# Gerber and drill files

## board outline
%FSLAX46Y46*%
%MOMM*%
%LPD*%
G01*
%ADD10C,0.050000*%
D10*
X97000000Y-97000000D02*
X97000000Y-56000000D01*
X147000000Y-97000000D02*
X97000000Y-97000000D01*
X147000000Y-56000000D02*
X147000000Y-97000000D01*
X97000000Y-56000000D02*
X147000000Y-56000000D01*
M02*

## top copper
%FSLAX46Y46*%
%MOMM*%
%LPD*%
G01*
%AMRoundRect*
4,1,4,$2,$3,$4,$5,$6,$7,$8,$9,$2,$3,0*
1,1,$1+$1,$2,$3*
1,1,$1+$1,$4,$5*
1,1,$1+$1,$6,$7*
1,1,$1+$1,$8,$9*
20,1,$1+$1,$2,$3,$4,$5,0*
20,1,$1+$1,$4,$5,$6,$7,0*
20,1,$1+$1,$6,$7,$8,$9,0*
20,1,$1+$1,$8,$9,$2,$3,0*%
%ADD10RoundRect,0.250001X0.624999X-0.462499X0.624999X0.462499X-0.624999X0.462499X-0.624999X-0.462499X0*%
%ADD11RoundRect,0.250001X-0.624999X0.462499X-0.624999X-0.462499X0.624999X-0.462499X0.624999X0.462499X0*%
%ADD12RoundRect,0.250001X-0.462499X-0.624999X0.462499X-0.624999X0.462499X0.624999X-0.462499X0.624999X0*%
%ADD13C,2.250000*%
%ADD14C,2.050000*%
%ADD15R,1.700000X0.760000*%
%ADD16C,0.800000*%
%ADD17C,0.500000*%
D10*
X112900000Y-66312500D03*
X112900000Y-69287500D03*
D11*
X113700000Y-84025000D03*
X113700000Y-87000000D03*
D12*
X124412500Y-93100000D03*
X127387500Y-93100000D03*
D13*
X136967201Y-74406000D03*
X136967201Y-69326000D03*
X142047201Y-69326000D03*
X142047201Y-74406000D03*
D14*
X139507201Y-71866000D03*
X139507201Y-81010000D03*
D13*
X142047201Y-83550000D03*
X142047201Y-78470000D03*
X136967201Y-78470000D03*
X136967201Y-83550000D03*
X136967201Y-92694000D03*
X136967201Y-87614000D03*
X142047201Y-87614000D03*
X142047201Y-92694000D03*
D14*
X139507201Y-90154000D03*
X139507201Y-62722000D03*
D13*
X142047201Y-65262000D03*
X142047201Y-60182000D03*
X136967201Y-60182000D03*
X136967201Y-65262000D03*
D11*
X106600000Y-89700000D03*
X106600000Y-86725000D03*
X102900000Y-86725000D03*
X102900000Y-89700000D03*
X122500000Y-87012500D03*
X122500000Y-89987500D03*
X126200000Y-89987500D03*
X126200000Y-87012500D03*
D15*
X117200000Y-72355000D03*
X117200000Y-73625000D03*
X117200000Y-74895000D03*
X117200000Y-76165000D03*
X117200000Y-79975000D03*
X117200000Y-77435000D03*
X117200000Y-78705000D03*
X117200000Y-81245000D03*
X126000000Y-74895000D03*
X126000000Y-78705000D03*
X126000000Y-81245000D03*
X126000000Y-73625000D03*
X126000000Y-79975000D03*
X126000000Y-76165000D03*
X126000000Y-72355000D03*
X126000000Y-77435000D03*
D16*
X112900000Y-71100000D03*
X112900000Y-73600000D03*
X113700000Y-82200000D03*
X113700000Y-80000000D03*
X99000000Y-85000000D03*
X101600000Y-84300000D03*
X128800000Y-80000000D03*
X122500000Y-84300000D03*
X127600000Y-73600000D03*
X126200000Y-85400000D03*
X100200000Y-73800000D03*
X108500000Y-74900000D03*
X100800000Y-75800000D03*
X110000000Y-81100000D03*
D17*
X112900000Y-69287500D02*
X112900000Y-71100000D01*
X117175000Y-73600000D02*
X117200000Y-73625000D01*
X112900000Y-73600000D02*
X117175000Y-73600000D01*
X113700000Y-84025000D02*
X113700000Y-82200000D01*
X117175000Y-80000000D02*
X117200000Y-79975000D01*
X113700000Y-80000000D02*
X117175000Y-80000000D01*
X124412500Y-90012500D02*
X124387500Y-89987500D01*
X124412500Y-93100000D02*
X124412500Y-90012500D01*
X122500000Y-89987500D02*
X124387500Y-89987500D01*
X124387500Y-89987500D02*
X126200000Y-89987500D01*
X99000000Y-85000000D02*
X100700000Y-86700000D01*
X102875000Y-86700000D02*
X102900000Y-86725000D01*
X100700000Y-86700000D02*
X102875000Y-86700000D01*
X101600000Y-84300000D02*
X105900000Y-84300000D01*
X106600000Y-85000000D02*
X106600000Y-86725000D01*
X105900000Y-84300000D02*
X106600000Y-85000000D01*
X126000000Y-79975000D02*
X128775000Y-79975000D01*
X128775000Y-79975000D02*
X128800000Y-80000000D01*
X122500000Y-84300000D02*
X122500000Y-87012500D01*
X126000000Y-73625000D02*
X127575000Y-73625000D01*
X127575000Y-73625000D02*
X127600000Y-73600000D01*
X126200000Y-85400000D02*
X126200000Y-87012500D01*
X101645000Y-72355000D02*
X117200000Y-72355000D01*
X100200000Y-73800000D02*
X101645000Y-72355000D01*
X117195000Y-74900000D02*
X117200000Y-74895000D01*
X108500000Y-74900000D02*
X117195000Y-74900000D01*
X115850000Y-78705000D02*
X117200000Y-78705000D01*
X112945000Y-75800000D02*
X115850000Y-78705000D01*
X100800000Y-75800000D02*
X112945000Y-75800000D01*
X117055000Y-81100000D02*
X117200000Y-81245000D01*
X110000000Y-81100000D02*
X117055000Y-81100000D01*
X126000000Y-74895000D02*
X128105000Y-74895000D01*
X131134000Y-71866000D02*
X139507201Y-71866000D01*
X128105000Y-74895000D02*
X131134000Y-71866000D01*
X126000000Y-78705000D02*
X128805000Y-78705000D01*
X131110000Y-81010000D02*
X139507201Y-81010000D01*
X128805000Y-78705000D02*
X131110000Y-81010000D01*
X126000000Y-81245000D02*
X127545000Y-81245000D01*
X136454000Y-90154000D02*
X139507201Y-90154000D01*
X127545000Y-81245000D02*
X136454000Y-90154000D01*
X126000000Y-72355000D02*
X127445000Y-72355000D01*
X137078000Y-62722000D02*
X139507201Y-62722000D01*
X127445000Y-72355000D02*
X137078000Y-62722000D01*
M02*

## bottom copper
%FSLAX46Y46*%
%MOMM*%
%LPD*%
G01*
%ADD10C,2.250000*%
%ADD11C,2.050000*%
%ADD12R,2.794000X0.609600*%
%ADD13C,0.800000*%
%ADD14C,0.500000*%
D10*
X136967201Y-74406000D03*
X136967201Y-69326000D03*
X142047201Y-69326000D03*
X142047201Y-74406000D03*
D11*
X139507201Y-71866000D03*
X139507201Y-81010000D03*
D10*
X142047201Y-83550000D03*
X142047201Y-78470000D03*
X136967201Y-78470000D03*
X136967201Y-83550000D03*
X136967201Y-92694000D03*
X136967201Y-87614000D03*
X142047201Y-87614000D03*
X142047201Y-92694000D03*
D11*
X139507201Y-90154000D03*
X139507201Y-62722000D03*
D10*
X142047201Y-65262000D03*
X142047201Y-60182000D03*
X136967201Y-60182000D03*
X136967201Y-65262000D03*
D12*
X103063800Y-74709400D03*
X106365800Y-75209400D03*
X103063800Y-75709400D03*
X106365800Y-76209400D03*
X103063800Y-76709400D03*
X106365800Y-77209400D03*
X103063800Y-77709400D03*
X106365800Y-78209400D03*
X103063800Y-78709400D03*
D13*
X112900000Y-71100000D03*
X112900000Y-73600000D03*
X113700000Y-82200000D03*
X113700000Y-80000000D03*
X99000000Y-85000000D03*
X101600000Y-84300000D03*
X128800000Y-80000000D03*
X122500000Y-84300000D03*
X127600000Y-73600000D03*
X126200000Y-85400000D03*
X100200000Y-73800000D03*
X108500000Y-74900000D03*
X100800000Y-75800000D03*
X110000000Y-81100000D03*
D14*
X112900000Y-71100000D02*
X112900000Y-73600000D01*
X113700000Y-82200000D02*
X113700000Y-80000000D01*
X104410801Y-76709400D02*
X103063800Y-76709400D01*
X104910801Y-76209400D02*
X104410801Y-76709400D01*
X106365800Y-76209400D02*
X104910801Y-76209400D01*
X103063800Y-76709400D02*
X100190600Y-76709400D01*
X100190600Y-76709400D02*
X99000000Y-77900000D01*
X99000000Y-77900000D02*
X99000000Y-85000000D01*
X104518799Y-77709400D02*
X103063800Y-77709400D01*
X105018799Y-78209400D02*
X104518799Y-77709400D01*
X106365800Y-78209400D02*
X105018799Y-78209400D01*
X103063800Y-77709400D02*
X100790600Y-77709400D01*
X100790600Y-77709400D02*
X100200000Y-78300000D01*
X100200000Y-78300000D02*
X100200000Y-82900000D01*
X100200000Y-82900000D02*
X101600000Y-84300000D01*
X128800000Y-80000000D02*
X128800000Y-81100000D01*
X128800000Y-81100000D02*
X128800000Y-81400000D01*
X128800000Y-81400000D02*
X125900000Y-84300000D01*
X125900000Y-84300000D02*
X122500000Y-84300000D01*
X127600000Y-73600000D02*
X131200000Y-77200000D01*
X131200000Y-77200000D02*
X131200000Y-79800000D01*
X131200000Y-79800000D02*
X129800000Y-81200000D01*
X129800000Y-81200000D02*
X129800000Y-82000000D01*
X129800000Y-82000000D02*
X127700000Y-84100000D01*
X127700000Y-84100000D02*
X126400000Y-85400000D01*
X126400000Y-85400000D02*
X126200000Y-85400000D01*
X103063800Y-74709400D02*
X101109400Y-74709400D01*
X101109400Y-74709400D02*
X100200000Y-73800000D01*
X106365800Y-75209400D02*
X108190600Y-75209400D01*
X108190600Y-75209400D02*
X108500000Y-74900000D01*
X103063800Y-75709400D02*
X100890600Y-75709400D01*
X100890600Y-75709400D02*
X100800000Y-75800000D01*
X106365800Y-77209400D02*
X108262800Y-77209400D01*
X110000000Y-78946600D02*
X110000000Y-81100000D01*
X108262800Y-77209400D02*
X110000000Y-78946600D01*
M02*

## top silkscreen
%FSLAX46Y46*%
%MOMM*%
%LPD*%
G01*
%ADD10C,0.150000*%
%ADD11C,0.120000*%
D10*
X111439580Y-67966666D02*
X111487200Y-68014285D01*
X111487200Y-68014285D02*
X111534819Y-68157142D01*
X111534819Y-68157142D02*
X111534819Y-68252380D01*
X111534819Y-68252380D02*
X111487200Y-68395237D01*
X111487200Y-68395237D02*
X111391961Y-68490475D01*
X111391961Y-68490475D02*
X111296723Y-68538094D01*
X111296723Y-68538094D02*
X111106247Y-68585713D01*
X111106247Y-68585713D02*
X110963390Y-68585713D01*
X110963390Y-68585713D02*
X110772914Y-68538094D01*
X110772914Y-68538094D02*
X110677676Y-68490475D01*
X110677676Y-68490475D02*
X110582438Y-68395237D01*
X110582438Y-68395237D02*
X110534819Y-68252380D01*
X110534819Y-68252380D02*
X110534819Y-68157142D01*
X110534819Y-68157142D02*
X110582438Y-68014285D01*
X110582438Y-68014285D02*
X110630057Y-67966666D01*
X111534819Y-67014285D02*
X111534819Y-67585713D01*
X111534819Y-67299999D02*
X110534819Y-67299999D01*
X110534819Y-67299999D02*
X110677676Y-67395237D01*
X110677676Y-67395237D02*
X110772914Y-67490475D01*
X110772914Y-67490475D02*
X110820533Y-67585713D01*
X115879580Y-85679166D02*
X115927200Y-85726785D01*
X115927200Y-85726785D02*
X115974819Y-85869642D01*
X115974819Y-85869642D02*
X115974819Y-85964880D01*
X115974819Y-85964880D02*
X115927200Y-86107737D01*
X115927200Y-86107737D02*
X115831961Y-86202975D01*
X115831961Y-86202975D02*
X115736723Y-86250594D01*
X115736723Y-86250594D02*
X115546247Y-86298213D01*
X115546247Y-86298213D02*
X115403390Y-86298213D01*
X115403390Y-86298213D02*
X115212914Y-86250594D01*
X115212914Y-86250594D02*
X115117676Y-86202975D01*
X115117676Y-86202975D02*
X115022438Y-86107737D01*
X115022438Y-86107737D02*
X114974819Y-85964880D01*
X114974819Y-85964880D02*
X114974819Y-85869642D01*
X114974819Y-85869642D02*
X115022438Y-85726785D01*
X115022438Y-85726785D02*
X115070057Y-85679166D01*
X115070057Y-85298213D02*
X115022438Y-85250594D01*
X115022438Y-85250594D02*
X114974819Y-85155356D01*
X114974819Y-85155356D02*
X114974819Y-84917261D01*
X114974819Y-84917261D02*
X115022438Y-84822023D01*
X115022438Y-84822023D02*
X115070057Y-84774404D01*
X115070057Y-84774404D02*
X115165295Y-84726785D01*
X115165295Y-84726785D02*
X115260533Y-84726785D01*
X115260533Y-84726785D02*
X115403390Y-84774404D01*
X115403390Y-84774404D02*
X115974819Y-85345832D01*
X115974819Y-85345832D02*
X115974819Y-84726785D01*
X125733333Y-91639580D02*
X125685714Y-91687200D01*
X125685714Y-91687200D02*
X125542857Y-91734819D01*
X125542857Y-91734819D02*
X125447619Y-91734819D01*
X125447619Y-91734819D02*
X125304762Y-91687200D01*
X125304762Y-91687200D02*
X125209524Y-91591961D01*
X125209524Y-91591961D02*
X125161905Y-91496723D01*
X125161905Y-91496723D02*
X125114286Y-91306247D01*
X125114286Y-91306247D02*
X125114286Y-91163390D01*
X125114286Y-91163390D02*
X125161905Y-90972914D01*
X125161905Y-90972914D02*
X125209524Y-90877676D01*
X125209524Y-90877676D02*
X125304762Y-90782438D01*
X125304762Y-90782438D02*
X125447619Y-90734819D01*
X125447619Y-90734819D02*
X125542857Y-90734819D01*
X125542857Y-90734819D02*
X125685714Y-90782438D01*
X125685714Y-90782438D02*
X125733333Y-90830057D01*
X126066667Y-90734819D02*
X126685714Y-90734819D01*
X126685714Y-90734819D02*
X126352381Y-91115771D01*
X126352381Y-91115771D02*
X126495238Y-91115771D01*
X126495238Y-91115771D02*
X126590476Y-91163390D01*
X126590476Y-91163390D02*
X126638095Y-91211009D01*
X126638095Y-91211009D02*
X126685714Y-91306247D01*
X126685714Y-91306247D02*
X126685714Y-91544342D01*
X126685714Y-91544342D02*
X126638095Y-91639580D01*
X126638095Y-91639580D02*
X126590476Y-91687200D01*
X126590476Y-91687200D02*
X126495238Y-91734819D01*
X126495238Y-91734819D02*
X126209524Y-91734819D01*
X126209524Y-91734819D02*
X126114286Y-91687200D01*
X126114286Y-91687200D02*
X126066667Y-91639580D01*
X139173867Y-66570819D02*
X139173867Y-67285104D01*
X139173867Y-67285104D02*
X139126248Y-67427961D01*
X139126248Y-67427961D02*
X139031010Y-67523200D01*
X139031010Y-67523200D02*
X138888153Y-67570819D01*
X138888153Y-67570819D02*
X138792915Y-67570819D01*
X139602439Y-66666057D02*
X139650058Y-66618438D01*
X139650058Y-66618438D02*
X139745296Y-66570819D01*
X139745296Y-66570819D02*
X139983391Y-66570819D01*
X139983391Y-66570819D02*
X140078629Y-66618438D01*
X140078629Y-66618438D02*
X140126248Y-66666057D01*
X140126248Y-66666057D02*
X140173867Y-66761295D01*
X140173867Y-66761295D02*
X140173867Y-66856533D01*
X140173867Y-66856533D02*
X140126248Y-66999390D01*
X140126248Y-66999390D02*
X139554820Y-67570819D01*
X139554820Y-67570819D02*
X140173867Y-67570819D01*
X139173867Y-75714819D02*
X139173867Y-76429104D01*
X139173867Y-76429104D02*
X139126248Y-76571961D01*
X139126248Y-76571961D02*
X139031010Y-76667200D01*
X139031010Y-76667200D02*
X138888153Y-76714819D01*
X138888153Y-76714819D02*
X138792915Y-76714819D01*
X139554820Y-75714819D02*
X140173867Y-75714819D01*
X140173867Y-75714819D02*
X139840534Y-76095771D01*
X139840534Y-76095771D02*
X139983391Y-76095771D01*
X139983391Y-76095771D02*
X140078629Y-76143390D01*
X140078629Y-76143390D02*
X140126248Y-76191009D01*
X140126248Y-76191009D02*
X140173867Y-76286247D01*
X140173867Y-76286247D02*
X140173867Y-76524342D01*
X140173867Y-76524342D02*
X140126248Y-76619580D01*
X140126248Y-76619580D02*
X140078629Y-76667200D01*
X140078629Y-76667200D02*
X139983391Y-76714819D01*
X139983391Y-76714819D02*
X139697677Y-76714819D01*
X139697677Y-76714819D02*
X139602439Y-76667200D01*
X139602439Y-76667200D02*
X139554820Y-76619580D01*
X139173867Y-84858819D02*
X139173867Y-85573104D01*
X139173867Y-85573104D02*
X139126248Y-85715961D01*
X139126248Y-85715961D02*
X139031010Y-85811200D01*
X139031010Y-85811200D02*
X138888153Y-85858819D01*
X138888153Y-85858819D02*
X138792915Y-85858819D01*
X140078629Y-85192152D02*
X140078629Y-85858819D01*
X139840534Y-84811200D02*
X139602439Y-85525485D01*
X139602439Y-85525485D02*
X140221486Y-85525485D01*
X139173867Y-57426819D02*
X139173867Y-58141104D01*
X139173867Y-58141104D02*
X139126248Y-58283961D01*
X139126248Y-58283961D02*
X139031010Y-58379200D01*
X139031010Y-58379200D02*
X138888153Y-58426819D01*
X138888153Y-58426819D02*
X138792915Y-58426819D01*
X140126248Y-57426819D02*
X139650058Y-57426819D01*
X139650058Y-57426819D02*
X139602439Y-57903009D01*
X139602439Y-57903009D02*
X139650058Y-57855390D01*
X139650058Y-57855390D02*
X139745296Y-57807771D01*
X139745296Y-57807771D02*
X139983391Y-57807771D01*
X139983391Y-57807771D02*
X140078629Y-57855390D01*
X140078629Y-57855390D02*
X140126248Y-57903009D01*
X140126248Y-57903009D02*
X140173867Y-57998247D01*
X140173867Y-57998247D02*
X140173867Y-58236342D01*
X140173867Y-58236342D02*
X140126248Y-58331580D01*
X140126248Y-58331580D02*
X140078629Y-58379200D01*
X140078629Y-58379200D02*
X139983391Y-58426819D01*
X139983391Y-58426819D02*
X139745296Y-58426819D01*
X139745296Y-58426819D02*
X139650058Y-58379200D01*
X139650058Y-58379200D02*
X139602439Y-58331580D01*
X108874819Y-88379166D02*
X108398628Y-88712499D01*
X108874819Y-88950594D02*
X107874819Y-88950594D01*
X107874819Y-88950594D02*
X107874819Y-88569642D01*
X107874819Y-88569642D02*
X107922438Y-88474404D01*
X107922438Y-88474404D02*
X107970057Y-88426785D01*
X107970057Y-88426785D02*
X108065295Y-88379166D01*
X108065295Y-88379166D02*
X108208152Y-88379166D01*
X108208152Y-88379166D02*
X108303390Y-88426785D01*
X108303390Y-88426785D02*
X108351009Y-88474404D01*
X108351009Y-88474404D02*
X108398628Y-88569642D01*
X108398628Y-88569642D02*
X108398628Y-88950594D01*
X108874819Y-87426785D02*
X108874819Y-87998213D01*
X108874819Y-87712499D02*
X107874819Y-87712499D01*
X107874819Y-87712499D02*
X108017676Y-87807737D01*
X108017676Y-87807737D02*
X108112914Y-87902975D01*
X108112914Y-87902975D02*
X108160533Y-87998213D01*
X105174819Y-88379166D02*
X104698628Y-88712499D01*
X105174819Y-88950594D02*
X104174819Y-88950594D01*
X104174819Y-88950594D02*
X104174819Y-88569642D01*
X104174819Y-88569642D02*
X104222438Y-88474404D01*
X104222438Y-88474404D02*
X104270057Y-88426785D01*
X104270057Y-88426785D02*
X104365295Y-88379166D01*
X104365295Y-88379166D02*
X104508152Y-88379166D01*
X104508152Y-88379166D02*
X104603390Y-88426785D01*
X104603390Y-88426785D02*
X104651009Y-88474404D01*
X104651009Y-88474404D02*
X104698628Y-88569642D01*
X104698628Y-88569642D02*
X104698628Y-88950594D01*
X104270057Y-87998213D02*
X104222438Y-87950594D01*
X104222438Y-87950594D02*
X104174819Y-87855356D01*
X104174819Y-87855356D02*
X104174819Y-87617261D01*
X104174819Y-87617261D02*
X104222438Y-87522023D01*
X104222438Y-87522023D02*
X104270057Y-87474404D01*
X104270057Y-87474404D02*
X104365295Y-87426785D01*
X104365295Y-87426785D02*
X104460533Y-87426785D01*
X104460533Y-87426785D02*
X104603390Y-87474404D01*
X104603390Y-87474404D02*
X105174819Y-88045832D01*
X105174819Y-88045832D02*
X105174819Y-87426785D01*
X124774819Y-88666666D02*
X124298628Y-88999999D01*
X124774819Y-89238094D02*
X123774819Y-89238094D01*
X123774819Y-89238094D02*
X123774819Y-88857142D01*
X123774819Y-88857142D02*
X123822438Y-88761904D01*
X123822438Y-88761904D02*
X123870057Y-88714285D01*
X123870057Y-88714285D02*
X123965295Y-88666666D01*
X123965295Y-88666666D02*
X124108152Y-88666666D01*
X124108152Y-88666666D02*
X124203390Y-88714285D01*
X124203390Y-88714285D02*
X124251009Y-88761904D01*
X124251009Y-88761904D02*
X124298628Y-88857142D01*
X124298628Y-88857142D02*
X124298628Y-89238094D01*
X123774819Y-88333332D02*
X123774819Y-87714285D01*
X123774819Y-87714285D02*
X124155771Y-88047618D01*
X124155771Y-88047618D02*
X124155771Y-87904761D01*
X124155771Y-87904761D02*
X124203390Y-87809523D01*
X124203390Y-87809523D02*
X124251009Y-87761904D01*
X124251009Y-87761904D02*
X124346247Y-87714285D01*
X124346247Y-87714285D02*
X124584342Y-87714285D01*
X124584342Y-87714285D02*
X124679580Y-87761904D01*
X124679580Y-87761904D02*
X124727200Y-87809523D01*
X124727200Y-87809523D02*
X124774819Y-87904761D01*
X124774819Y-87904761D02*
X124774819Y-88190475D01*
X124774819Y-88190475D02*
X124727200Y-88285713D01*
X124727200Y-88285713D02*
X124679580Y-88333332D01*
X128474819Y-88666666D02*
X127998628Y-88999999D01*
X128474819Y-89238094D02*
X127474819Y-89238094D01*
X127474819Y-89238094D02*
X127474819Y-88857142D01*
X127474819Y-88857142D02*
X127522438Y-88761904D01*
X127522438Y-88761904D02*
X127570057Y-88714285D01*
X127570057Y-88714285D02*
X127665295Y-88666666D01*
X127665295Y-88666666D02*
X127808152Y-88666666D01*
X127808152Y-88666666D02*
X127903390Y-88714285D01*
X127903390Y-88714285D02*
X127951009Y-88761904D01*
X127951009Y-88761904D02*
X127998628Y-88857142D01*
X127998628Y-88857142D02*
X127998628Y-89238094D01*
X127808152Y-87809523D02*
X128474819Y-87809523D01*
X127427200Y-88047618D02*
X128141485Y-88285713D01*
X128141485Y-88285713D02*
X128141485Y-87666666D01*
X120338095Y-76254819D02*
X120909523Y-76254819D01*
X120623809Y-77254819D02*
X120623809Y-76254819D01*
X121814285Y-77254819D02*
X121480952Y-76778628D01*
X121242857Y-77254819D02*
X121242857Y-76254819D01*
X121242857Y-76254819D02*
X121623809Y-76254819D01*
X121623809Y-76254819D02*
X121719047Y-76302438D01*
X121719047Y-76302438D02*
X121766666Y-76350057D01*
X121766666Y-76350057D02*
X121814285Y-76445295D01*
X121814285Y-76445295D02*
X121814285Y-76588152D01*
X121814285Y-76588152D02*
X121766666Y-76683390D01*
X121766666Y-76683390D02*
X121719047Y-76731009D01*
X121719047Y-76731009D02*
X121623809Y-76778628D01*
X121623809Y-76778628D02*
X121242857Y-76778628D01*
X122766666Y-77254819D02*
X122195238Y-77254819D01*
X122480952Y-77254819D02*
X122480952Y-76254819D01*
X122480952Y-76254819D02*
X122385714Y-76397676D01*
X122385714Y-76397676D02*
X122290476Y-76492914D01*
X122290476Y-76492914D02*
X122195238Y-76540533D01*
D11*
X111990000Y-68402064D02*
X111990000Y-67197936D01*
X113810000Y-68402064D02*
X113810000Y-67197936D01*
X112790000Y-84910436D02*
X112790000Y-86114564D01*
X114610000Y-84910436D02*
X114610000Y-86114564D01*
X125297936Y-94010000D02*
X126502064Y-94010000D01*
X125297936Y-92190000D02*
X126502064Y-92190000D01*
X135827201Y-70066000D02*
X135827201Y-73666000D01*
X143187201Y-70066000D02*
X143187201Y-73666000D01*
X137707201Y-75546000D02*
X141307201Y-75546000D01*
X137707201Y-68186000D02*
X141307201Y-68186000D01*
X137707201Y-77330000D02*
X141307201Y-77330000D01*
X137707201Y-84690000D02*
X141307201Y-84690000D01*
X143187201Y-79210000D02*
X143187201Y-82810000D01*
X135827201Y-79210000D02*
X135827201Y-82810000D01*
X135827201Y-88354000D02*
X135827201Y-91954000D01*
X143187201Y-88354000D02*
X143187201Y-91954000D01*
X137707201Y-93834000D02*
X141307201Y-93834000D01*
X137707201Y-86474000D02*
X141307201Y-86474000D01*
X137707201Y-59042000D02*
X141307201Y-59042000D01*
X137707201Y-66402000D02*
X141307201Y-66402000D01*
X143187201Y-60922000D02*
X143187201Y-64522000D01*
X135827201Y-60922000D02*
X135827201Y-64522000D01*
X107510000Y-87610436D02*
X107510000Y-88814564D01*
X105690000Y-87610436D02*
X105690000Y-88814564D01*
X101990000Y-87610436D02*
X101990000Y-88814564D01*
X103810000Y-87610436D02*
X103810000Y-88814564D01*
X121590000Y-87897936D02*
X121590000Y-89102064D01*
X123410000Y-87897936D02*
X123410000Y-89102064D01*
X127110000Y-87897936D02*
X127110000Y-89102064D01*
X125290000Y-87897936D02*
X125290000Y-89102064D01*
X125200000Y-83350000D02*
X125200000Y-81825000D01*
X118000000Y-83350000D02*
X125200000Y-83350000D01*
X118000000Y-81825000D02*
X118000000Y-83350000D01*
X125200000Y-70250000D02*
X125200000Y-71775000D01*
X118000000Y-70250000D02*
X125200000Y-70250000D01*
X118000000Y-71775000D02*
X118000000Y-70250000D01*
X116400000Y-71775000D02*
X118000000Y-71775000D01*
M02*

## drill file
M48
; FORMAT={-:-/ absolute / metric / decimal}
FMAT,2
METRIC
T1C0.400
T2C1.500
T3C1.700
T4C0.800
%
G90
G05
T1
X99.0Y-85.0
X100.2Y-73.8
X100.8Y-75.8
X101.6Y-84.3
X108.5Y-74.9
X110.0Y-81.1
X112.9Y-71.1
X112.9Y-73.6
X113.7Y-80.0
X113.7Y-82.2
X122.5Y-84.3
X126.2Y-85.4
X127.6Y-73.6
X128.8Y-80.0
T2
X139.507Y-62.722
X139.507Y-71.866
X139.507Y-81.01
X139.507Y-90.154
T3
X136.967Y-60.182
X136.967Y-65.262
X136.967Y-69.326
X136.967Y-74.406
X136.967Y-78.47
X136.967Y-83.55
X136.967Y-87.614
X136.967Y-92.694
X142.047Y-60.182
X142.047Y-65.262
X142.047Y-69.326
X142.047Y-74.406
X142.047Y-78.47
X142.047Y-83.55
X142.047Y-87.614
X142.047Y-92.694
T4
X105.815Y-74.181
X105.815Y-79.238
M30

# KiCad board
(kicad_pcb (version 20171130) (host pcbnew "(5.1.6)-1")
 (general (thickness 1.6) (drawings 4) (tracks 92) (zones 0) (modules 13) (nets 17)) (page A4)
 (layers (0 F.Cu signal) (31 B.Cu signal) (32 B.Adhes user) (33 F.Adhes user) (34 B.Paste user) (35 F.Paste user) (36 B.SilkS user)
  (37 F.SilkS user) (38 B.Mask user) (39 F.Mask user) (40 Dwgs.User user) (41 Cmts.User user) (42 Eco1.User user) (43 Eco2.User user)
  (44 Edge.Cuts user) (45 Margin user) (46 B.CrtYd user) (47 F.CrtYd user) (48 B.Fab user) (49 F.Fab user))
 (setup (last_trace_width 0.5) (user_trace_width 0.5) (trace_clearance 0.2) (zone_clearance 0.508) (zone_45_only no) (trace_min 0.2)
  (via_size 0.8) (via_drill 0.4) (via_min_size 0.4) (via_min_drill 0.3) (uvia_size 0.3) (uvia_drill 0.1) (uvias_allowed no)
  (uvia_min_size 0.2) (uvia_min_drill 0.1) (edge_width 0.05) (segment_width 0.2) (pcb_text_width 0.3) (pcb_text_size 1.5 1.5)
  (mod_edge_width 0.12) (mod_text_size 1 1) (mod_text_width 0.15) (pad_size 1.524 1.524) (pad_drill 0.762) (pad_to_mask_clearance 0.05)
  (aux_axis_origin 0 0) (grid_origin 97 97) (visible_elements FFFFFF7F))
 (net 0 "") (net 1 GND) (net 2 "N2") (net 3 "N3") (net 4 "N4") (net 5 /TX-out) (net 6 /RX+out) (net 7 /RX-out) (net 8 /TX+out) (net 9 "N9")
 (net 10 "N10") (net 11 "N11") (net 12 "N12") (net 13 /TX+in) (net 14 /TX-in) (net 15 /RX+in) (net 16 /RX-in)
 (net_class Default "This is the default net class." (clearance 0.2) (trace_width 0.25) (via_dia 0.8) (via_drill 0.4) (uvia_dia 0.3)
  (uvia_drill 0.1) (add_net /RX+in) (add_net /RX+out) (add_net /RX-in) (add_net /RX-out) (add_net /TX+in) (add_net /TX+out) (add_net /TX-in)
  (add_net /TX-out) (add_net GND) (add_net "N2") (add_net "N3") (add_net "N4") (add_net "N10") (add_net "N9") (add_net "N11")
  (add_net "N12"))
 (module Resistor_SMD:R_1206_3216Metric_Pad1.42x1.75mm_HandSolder (layer F.Cu) (at 112.9 67.8 90)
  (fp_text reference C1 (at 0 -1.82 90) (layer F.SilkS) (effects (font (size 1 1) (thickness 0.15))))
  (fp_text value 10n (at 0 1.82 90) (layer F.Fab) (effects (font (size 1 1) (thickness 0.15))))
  (fp_line (start -0.602064 -0.91) (end 0.602064 -0.91) (layer F.SilkS) (width 0.12))
  (fp_line (start -0.602064 0.91) (end 0.602064 0.91) (layer F.SilkS) (width 0.12))
  (pad 2 smd roundrect (at 1.4875 0 90) (size 1.425 1.75) (layers F.Cu F.Paste F.Mask) (roundrect_rratio 0.175439) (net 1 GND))
  (pad 1 smd roundrect (at -1.4875 0 90) (size 1.425 1.75) (layers F.Cu F.Paste F.Mask) (roundrect_rratio 0.175439) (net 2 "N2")))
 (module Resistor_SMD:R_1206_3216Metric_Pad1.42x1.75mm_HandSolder (layer F.Cu) (at 113.7 85.5125 270)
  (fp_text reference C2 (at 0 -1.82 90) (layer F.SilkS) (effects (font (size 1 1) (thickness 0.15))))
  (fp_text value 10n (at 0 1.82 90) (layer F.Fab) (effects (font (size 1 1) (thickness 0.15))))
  (fp_line (start -0.602064 0.91) (end 0.602064 0.91) (layer F.SilkS) (width 0.12))
  (fp_line (start -0.602064 -0.91) (end 0.602064 -0.91) (layer F.SilkS) (width 0.12))
  (pad 1 smd roundrect (at -1.4875 0 270) (size 1.425 1.75) (layers F.Cu F.Paste F.Mask) (roundrect_rratio 0.175439) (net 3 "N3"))
  (pad 2 smd roundrect (at 1.4875 0 270) (size 1.425 1.75) (layers F.Cu F.Paste F.Mask) (roundrect_rratio 0.175439) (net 1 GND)))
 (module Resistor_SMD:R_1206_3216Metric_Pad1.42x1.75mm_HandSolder (layer F.Cu) (at 125.9 93.1)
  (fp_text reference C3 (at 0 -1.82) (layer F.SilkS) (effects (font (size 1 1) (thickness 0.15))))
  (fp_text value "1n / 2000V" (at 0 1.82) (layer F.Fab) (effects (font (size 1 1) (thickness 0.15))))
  (fp_line (start -0.602064 0.91) (end 0.602064 0.91) (layer F.SilkS) (width 0.12))
  (fp_line (start -0.602064 -0.91) (end 0.602064 -0.91) (layer F.SilkS) (width 0.12))
  (pad 1 smd roundrect (at -1.4875 0) (size 1.425 1.75) (layers F.Cu F.Paste F.Mask) (roundrect_rratio 0.175439) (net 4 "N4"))
  (pad 2 smd roundrect (at 1.4875 0) (size 1.425 1.75) (layers F.Cu F.Paste F.Mask) (roundrect_rratio 0.175439) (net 1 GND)))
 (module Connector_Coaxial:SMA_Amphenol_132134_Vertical (layer F.Cu) (at 139.507201 71.866)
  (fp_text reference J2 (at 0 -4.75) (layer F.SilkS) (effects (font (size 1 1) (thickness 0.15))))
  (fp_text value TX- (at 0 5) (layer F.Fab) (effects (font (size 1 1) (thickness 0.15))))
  (fp_line (start -3.68 -1.8) (end -3.68 1.8) (layer F.SilkS) (width 0.12))
  (fp_line (start 3.68 -1.8) (end 3.68 1.8) (layer F.SilkS) (width 0.12))
  (fp_line (start -1.8 3.68) (end 1.8 3.68) (layer F.SilkS) (width 0.12))
  (fp_line (start -1.8 -3.68) (end 1.8 -3.68) (layer F.SilkS) (width 0.12))
  (pad 2 thru_hole circle (at -2.54 2.54) (size 2.25 2.25) (drill 1.7) (layers *.Cu *.Mask) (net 1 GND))
  (pad 2 thru_hole circle (at -2.54 -2.54) (size 2.25 2.25) (drill 1.7) (layers *.Cu *.Mask) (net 1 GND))
  (pad 2 thru_hole circle (at 2.54 -2.54) (size 2.25 2.25) (drill 1.7) (layers *.Cu *.Mask) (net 1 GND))
  (pad 2 thru_hole circle (at 2.54 2.54) (size 2.25 2.25) (drill 1.7) (layers *.Cu *.Mask) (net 1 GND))
  (pad 1 thru_hole circle (at 0 0) (size 2.05 2.05) (drill 1.5) (layers *.Cu *.Mask) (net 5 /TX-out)))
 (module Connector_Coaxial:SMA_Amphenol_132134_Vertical (layer F.Cu) (at 139.507201 81.01)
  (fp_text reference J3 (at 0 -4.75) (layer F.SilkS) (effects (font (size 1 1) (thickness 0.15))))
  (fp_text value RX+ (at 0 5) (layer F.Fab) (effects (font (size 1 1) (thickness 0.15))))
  (fp_line (start -1.8 -3.68) (end 1.8 -3.68) (layer F.SilkS) (width 0.12))
  (fp_line (start -1.8 3.68) (end 1.8 3.68) (layer F.SilkS) (width 0.12))
  (fp_line (start 3.68 -1.8) (end 3.68 1.8) (layer F.SilkS) (width 0.12))
  (fp_line (start -3.68 -1.8) (end -3.68 1.8) (layer F.SilkS) (width 0.12))
  (pad 1 thru_hole circle (at 0 0) (size 2.05 2.05) (drill 1.5) (layers *.Cu *.Mask) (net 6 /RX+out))
  (pad 2 thru_hole circle (at 2.54 2.54) (size 2.25 2.25) (drill 1.7) (layers *.Cu *.Mask) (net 1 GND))
  (pad 2 thru_hole circle (at 2.54 -2.54) (size 2.25 2.25) (drill 1.7) (layers *.Cu *.Mask) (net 1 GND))
  (pad 2 thru_hole circle (at -2.54 -2.54) (size 2.25 2.25) (drill 1.7) (layers *.Cu *.Mask) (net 1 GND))
  (pad 2 thru_hole circle (at -2.54 2.54) (size 2.25 2.25) (drill 1.7) (layers *.Cu *.Mask) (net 1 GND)))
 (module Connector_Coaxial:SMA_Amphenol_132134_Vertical (layer F.Cu) (at 139.507201 90.154)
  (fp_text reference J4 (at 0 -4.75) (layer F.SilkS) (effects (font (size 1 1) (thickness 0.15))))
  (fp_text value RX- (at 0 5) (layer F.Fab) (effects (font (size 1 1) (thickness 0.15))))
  (fp_line (start -3.68 -1.8) (end -3.68 1.8) (layer F.SilkS) (width 0.12))
  (fp_line (start 3.68 -1.8) (end 3.68 1.8) (layer F.SilkS) (width 0.12))
  (fp_line (start -1.8 3.68) (end 1.8 3.68) (layer F.SilkS) (width 0.12))
  (fp_line (start -1.8 -3.68) (end 1.8 -3.68) (layer F.SilkS) (width 0.12))
  (pad 2 thru_hole circle (at -2.54 2.54) (size 2.25 2.25) (drill 1.7) (layers *.Cu *.Mask) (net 1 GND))
  (pad 2 thru_hole circle (at -2.54 -2.54) (size 2.25 2.25) (drill 1.7) (layers *.Cu *.Mask) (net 1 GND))
  (pad 2 thru_hole circle (at 2.54 -2.54) (size 2.25 2.25) (drill 1.7) (layers *.Cu *.Mask) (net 1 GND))
  (pad 2 thru_hole circle (at 2.54 2.54) (size 2.25 2.25) (drill 1.7) (layers *.Cu *.Mask) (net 1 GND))
  (pad 1 thru_hole circle (at 0 0) (size 2.05 2.05) (drill 1.5) (layers *.Cu *.Mask) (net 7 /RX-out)))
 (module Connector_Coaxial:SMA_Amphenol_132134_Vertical (layer F.Cu) (at 139.507201 62.722)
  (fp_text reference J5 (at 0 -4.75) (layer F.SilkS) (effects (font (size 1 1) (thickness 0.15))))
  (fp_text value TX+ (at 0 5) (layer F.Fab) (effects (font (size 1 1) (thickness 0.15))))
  (fp_line (start -1.8 -3.68) (end 1.8 -3.68) (layer F.SilkS) (width 0.12))
  (fp_line (start -1.8 3.68) (end 1.8 3.68) (layer F.SilkS) (width 0.12))
  (fp_line (start 3.68 -1.8) (end 3.68 1.8) (layer F.SilkS) (width 0.12))
  (fp_line (start -3.68 -1.8) (end -3.68 1.8) (layer F.SilkS) (width 0.12))
  (pad 1 thru_hole circle (at 0 0) (size 2.05 2.05) (drill 1.5) (layers *.Cu *.Mask) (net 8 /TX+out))
  (pad 2 thru_hole circle (at 2.54 2.54) (size 2.25 2.25) (drill 1.7) (layers *.Cu *.Mask) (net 1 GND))
  (pad 2 thru_hole circle (at 2.54 -2.54) (size 2.25 2.25) (drill 1.7) (layers *.Cu *.Mask) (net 1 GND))
  (pad 2 thru_hole circle (at -2.54 -2.54) (size 2.25 2.25) (drill 1.7) (layers *.Cu *.Mask) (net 1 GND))
  (pad 2 thru_hole circle (at -2.54 2.54) (size 2.25 2.25) (drill 1.7) (layers *.Cu *.Mask) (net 1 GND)))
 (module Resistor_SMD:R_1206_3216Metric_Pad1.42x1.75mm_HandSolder (layer F.Cu) (at 106.6 88.2125 270)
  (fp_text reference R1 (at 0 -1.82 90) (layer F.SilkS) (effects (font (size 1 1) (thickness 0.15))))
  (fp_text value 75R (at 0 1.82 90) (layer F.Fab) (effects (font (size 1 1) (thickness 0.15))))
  (fp_line (start -0.602064 -0.91) (end 0.602064 -0.91) (layer F.SilkS) (width 0.12))
  (fp_line (start -0.602064 0.91) (end 0.602064 0.91) (layer F.SilkS) (width 0.12))
  (pad 2 smd roundrect (at 1.4875 0 270) (size 1.425 1.75) (layers F.Cu F.Paste F.Mask) (roundrect_rratio 0.175439) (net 1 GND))
  (pad 1 smd roundrect (at -1.4875 0 270) (size 1.425 1.75) (layers F.Cu F.Paste F.Mask) (roundrect_rratio 0.175439) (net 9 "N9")))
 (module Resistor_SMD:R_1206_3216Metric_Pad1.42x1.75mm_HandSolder (layer F.Cu) (at 102.9 88.2125 270)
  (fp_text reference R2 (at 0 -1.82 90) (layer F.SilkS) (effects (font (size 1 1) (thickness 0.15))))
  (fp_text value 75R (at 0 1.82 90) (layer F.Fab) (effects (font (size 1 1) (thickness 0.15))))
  (fp_line (start -0.602064 0.91) (end 0.602064 0.91) (layer F.SilkS) (width 0.12))
  (fp_line (start -0.602064 -0.91) (end 0.602064 -0.91) (layer F.SilkS) (width 0.12))
  (pad 1 smd roundrect (at -1.4875 0 270) (size 1.425 1.75) (layers F.Cu F.Paste F.Mask) (roundrect_rratio 0.175439) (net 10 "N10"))
  (pad 2 smd roundrect (at 1.4875 0 270) (size 1.425 1.75) (layers F.Cu F.Paste F.Mask) (roundrect_rratio 0.175439) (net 1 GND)))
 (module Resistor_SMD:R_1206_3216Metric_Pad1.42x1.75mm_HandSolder (layer F.Cu) (at 122.5 88.5 270)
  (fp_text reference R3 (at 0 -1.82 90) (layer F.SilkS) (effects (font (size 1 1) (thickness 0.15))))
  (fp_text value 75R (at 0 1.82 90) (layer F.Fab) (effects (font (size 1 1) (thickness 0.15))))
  (fp_line (start -0.602064 0.91) (end 0.602064 0.91) (layer F.SilkS) (width 0.12))
  (fp_line (start -0.602064 -0.91) (end 0.602064 -0.91) (layer F.SilkS) (width 0.12))
  (pad 1 smd roundrect (at -1.4875 0 270) (size 1.425 1.75) (layers F.Cu F.Paste F.Mask) (roundrect_rratio 0.175439) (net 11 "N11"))
  (pad 2 smd roundrect (at 1.4875 0 270) (size 1.425 1.75) (layers F.Cu F.Paste F.Mask) (roundrect_rratio 0.175439) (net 4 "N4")))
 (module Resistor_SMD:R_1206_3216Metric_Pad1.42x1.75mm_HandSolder (layer F.Cu) (at 126.2 88.5 270)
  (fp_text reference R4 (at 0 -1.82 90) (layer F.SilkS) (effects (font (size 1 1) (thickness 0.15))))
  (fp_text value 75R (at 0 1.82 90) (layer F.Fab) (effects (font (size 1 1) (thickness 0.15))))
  (fp_line (start -0.602064 -0.91) (end 0.602064 -0.91) (layer F.SilkS) (width 0.12))
  (fp_line (start -0.602064 0.91) (end 0.602064 0.91) (layer F.SilkS) (width 0.12))
  (pad 2 smd roundrect (at 1.4875 0 270) (size 1.425 1.75) (layers F.Cu F.Paste F.Mask) (roundrect_rratio 0.175439) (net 4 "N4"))
  (pad 1 smd roundrect (at -1.4875 0 270) (size 1.425 1.75) (layers F.Cu F.Paste F.Mask) (roundrect_rratio 0.175439) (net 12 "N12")))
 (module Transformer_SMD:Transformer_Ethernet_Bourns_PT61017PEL (layer F.Cu) (at 121.6 76.8)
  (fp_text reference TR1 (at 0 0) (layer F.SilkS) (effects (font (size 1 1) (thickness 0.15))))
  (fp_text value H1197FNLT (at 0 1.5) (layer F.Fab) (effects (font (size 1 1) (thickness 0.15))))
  (fp_line (start 3.6 6.55) (end 3.6 5.025) (layer F.SilkS) (width 0.12))
  (fp_line (start -3.6 6.55) (end 3.6 6.55) (layer F.SilkS) (width 0.12))
  (fp_line (start -3.6 5.025) (end -3.6 6.55) (layer F.SilkS) (width 0.12))
  (fp_line (start 3.6 -6.55) (end 3.6 -5.025) (layer F.SilkS) (width 0.12))
  (fp_line (start -3.6 -6.55) (end 3.6 -6.55) (layer F.SilkS) (width 0.12))
  (fp_line (start -3.6 -5.025) (end -3.6 -6.55) (layer F.SilkS) (width 0.12))
  (fp_line (start -5.2 -5.025) (end -3.6 -5.025) (layer F.SilkS) (width 0.12))
  (pad 1 smd rect (at -4.4 -4.445) (size 1.7 0.76) (layers F.Cu F.Paste F.Mask) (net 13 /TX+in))
  (pad 2 smd rect (at -4.4 -3.175) (size 1.7 0.76) (layers F.Cu F.Paste F.Mask) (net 2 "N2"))
  (pad 3 smd rect (at -4.4 -1.905) (size 1.7 0.76) (layers F.Cu F.Paste F.Mask) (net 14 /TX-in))
  (pad 4 smd rect (at -4.4 -0.635) (size 1.7 0.76) (layers F.Cu F.Paste F.Mask))
  (pad 7 smd rect (at -4.4 3.175) (size 1.7 0.76) (layers F.Cu F.Paste F.Mask) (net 3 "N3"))
  (pad 5 smd rect (at -4.4 0.635) (size 1.7 0.76) (layers F.Cu F.Paste F.Mask))
  (pad 6 smd rect (at -4.4 1.905) (size 1.7 0.76) (layers F.Cu F.Paste F.Mask) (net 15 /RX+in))
  (pad 8 smd rect (at -4.4 4.445) (size 1.7 0.76) (layers F.Cu F.Paste F.Mask) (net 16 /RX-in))
  (pad 14 smd rect (at 4.4 -1.905) (size 1.7 0.76) (layers F.Cu F.Paste F.Mask) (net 5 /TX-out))
  (pad 11 smd rect (at 4.4 1.905) (size 1.7 0.76) (layers F.Cu F.Paste F.Mask) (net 6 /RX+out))
  (pad 9 smd rect (at 4.4 4.445) (size 1.7 0.76) (layers F.Cu F.Paste F.Mask) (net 7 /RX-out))
  (pad 15 smd rect (at 4.4 -3.175) (size 1.7 0.76) (layers F.Cu F.Paste F.Mask) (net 12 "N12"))
  (pad 10 smd rect (at 4.4 3.175) (size 1.7 0.76) (layers F.Cu F.Paste F.Mask) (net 11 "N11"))
  (pad 13 smd rect (at 4.4 -0.635) (size 1.7 0.76) (layers F.Cu F.Paste F.Mask))
  (pad 16 smd rect (at 4.4 -4.445) (size 1.7 0.76) (layers F.Cu F.Paste F.Mask) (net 8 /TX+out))
  (pad 12 smd rect (at 4.4 0.635) (size 1.7 0.76) (layers F.Cu F.Paste F.Mask)))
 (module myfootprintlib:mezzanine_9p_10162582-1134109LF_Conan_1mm (layer B.Cu) (at 114.0638 90.7094 270)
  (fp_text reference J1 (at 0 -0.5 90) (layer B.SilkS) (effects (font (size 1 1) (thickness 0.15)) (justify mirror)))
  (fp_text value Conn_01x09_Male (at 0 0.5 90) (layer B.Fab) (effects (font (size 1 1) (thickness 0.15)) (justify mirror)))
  (pad 1 smd rect (at -16 11 270) (size 0.6096 2.794) (layers B.Cu B.Paste B.Mask) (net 13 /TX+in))
  (pad 2 smd rect (at -15.5 7.698 270) (size 0.6096 2.794) (layers B.Cu B.Paste B.Mask) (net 14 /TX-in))
  (pad 3 smd rect (at -15 11 270) (size 0.6096 2.794) (layers B.Cu B.Paste B.Mask) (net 15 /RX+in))
  (pad 4 smd rect (at -14.5 7.698 270) (size 0.6096 2.794) (layers B.Cu B.Paste B.Mask) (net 10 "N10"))
  (pad 5 smd rect (at -14 11 270) (size 0.6096 2.794) (layers B.Cu B.Paste B.Mask) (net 10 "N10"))
  (pad 6 smd rect (at -13.5 7.698 270) (size 0.6096 2.794) (layers B.Cu B.Paste B.Mask) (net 16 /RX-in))
  (pad 7 smd rect (at -13 11 270) (size 0.6096 2.794) (layers B.Cu B.Paste B.Mask) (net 9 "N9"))
  (pad 8 smd rect (at -12.5 7.698 270) (size 0.6096 2.794) (layers B.Cu B.Paste B.Mask) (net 9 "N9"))
  (pad 9 smd rect (at -12 11 270) (size 0.6096 2.794) (layers B.Cu B.Paste B.Mask) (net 1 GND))
  (pad 10 smd rect (at -17.7225 9.349 270) (size 1.397 6.096) (layers B.Paste))
  (pad 11 smd rect (at -10.2775 9.349 270) (size 1.397 6.096) (layers B.Paste))
  (pad "" np_thru_hole circle (at -16.5287 8.24918 270) (size 0.8 0.8) (drill 0.8) (layers *.Cu *.Mask))
  (pad "" np_thru_hole circle (at -11.4713 8.24918 270) (size 0.8 0.8) (drill 0.8) (layers *.Cu *.Mask)))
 (gr_line (start 97 97) (end 97 56) (layer Edge.Cuts) (width 0.05))
 (gr_line (start 147 97) (end 97 97) (layer Edge.Cuts) (width 0.05))
 (gr_line (start 147 56) (end 147 97) (layer Edge.Cuts) (width 0.05))
 (gr_line (start 97 56) (end 147 56) (layer Edge.Cuts) (width 0.05))
 (via (at 112.9 71.1) (size 0.8) (drill 0.4) (layers F.Cu B.Cu) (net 2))
 (segment (start 112.9 69.2875) (end 112.9 71.1) (width 0.5) (layer F.Cu) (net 2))
 (via (at 112.9 73.6) (size 0.8) (drill 0.4) (layers F.Cu B.Cu) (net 2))
 (segment (start 112.9 71.1) (end 112.9 73.6) (width 0.5) (layer B.Cu) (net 2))
 (segment (start 117.175 73.6) (end 117.2 73.625) (width 0.5) (layer F.Cu) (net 2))
 (segment (start 112.9 73.6) (end 117.175 73.6) (width 0.5) (layer F.Cu) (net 2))
 (via (at 113.7 82.2) (size 0.8) (drill 0.4) (layers F.Cu B.Cu) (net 3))
 (segment (start 113.7 84.025) (end 113.7 82.2) (width 0.5) (layer F.Cu) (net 3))
 (via (at 113.7 80) (size 0.8) (drill 0.4) (layers F.Cu B.Cu) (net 3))
 (segment (start 113.7 82.2) (end 113.7 80) (width 0.5) (layer B.Cu) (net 3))
 (segment (start 117.175 80) (end 117.2 79.975) (width 0.5) (layer F.Cu) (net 3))
 (segment (start 113.7 80) (end 117.175 80) (width 0.5) (layer F.Cu) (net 3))
 (segment (start 124.4125 90.0125) (end 124.3875 89.9875) (width 0.5) (layer F.Cu) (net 4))
 (segment (start 124.4125 93.1) (end 124.4125 90.0125) (width 0.5) (layer F.Cu) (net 4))
 (segment (start 122.5 89.9875) (end 124.3875 89.9875) (width 0.5) (layer F.Cu) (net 4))
 (segment (start 124.3875 89.9875) (end 126.2 89.9875) (width 0.5) (layer F.Cu) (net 4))
 (segment (start 104.410801 76.7094) (end 103.0638 76.7094) (width 0.5) (layer B.Cu) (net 10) (status 30))
 (segment (start 104.910801 76.2094) (end 104.410801 76.7094) (width 0.5) (layer B.Cu) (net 10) (status 20))
 (segment (start 106.3658 76.2094) (end 104.910801 76.2094) (width 0.5) (layer B.Cu) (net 10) (status 10))
 (segment (start 103.0638 76.7094) (end 100.1906 76.7094) (width 0.5) (layer B.Cu) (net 10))
 (segment (start 100.1906 76.7094) (end 99 77.9) (width 0.5) (layer B.Cu) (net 10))
 (via (at 99 85) (size 0.8) (drill 0.4) (layers F.Cu B.Cu) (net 10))
 (segment (start 99 77.9) (end 99 85) (width 0.5) (layer B.Cu) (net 10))
 (segment (start 99 85) (end 100.7 86.7) (width 0.5) (layer F.Cu) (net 10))
 (segment (start 102.875 86.7) (end 102.9 86.725) (width 0.5) (layer F.Cu) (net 10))
 (segment (start 100.7 86.7) (end 102.875 86.7) (width 0.5) (layer F.Cu) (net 10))
 (segment (start 104.518799 77.7094) (end 103.0638 77.7094) (width 0.5) (layer B.Cu) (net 9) (status 20))
 (segment (start 105.018799 78.2094) (end 104.518799 77.7094) (width 0.5) (layer B.Cu) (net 9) (status 10))
 (segment (start 106.3658 78.2094) (end 105.018799 78.2094) (width 0.5) (layer B.Cu) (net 9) (status 30))
 (segment (start 103.0638 77.7094) (end 100.7906 77.7094) (width 0.5) (layer B.Cu) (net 9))
 (segment (start 100.7906 77.7094) (end 100.2 78.3) (width 0.5) (layer B.Cu) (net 9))
 (segment (start 100.2 78.3) (end 100.2 82.9) (width 0.5) (layer B.Cu) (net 9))
 (via (at 101.6 84.3) (size 0.8) (drill 0.4) (layers F.Cu B.Cu) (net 9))
 (segment (start 100.2 82.9) (end 101.6 84.3) (width 0.5) (layer B.Cu) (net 9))
 (segment (start 101.6 84.3) (end 105.9 84.3) (width 0.5) (layer F.Cu) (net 9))
 (segment (start 106.6 85) (end 106.6 86.725) (width 0.5) (layer F.Cu) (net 9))
 (segment (start 105.9 84.3) (end 106.6 85) (width 0.5) (layer F.Cu) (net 9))
 (via (at 128.8 80) (size 0.8) (drill 0.4) (layers F.Cu B.Cu) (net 11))
 (segment (start 126 79.975) (end 128.775 79.975) (width 0.5) (layer F.Cu) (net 11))
 (segment (start 128.775 79.975) (end 128.8 80) (width 0.5) (layer F.Cu) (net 11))
 (segment (start 128.8 80) (end 128.8 81.1) (width 0.5) (layer B.Cu) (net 11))
 (segment (start 128.8 81.1) (end 128.8 81.4) (width 0.5) (layer B.Cu) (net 11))
 (segment (start 128.8 81.4) (end 125.9 84.3) (width 0.5) (layer B.Cu) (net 11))
 (via (at 122.5 84.3) (size 0.8) (drill 0.4) (layers F.Cu B.Cu) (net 11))
 (segment (start 125.9 84.3) (end 122.5 84.3) (width 0.5) (layer B.Cu) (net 11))
 (segment (start 122.5 84.3) (end 122.5 87.0125) (width 0.5) (layer F.Cu) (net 11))
 (via (at 127.6 73.6) (size 0.8) (drill 0.4) (layers F.Cu B.Cu) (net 12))
 (segment (start 126 73.625) (end 127.575 73.625) (width 0.5) (layer F.Cu) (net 12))
 (segment (start 127.575 73.625) (end 127.6 73.6) (width 0.5) (layer F.Cu) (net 12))
 (segment (start 127.6 73.6) (end 131.2 77.2) (width 0.5) (layer B.Cu) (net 12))
 (segment (start 131.2 77.2) (end 131.2 79.8) (width 0.5) (layer B.Cu) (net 12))
 (segment (start 131.2 79.8) (end 129.8 81.2) (width 0.5) (layer B.Cu) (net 12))
 (segment (start 129.8 81.2) (end 129.8 82) (width 0.5) (layer B.Cu) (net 12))
 (segment (start 129.8 82) (end 127.7 84.1) (width 0.5) (layer B.Cu) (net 12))
 (via (at 126.2 85.4) (size 0.8) (drill 0.4) (layers F.Cu B.Cu) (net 12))
 (segment (start 127.7 84.1) (end 126.4 85.4) (width 0.5) (layer B.Cu) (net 12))
 (segment (start 126.4 85.4) (end 126.2 85.4) (width 0.5) (layer B.Cu) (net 12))
 (segment (start 126.2 85.4) (end 126.2 87.0125) (width 0.5) (layer F.Cu) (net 12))
 (via (at 100.2 73.8) (size 0.8) (drill 0.4) (layers F.Cu B.Cu) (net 13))
 (segment (start 103.0638 74.7094) (end 101.1094 74.7094) (width 0.5) (layer B.Cu) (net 13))
 (segment (start 101.1094 74.7094) (end 100.2 73.8) (width 0.5) (layer B.Cu) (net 13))
 (segment (start 101.645 72.355) (end 117.2 72.355) (width 0.5) (layer F.Cu) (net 13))
 (segment (start 100.2 73.8) (end 101.645 72.355) (width 0.5) (layer F.Cu) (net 13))
 (via (at 108.5 74.9) (size 0.8) (drill 0.4) (layers F.Cu B.Cu) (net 14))
 (segment (start 106.3658 75.2094) (end 108.1906 75.2094) (width 0.5) (layer B.Cu) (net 14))
 (segment (start 108.1906 75.2094) (end 108.5 74.9) (width 0.5) (layer B.Cu) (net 14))
 (segment (start 117.195 74.9) (end 117.2 74.895) (width 0.5) (layer F.Cu) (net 14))
 (segment (start 108.5 74.9) (end 117.195 74.9) (width 0.5) (layer F.Cu) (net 14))
 (via (at 100.8 75.8) (size 0.8) (drill 0.4) (layers F.Cu B.Cu) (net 15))
 (segment (start 103.0638 75.7094) (end 100.8906 75.7094) (width 0.5) (layer B.Cu) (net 15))
 (segment (start 100.8906 75.7094) (end 100.8 75.8) (width 0.5) (layer B.Cu) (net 15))
 (segment (start 115.85 78.705) (end 117.2 78.705) (width 0.5) (layer F.Cu) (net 15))
 (segment (start 112.945 75.8) (end 115.85 78.705) (width 0.5) (layer F.Cu) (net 15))
 (segment (start 100.8 75.8) (end 112.945 75.8) (width 0.5) (layer F.Cu) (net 15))
 (via (at 110 81.1) (size 0.8) (drill 0.4) (layers F.Cu B.Cu) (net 16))
 (segment (start 106.3658 77.2094) (end 108.2628 77.2094) (width 0.5) (layer B.Cu) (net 16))
 (segment (start 110 78.9466) (end 110 81.1) (width 0.5) (layer B.Cu) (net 16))
 (segment (start 108.2628 77.2094) (end 110 78.9466) (width 0.5) (layer B.Cu) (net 16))
 (segment (start 117.055 81.1) (end 117.2 81.245) (width 0.5) (layer F.Cu) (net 16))
 (segment (start 110 81.1) (end 117.055 81.1) (width 0.5) (layer F.Cu) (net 16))
 (segment (start 126 74.895) (end 128.105 74.895) (width 0.5) (layer F.Cu) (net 5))
 (segment (start 131.134 71.866) (end 139.507201 71.866) (width 0.5) (layer F.Cu) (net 5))
 (segment (start 128.105 74.895) (end 131.134 71.866) (width 0.5) (layer F.Cu) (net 5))
 (segment (start 126 78.705) (end 128.805 78.705) (width 0.5) (layer F.Cu) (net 6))
 (segment (start 131.11 81.01) (end 139.507201 81.01) (width 0.5) (layer F.Cu) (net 6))
 (segment (start 128.805 78.705) (end 131.11 81.01) (width 0.5) (layer F.Cu) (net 6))
 (segment (start 126 81.245) (end 127.545 81.245) (width 0.5) (layer F.Cu) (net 7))
 (segment (start 136.454 90.154) (end 139.507201 90.154) (width 0.5) (layer F.Cu) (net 7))
 (segment (start 127.545 81.245) (end 136.454 90.154) (width 0.5) (layer F.Cu) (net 7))
 (segment (start 126 72.355) (end 127.445 72.355) (width 0.5) (layer F.Cu) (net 8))
 (segment (start 137.078 62.722) (end 139.507201 62.722) (width 0.5) (layer F.Cu) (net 8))
 (segment (start 127.445 72.355) (end 137.078 62.722) (width 0.5) (layer F.Cu) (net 8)))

